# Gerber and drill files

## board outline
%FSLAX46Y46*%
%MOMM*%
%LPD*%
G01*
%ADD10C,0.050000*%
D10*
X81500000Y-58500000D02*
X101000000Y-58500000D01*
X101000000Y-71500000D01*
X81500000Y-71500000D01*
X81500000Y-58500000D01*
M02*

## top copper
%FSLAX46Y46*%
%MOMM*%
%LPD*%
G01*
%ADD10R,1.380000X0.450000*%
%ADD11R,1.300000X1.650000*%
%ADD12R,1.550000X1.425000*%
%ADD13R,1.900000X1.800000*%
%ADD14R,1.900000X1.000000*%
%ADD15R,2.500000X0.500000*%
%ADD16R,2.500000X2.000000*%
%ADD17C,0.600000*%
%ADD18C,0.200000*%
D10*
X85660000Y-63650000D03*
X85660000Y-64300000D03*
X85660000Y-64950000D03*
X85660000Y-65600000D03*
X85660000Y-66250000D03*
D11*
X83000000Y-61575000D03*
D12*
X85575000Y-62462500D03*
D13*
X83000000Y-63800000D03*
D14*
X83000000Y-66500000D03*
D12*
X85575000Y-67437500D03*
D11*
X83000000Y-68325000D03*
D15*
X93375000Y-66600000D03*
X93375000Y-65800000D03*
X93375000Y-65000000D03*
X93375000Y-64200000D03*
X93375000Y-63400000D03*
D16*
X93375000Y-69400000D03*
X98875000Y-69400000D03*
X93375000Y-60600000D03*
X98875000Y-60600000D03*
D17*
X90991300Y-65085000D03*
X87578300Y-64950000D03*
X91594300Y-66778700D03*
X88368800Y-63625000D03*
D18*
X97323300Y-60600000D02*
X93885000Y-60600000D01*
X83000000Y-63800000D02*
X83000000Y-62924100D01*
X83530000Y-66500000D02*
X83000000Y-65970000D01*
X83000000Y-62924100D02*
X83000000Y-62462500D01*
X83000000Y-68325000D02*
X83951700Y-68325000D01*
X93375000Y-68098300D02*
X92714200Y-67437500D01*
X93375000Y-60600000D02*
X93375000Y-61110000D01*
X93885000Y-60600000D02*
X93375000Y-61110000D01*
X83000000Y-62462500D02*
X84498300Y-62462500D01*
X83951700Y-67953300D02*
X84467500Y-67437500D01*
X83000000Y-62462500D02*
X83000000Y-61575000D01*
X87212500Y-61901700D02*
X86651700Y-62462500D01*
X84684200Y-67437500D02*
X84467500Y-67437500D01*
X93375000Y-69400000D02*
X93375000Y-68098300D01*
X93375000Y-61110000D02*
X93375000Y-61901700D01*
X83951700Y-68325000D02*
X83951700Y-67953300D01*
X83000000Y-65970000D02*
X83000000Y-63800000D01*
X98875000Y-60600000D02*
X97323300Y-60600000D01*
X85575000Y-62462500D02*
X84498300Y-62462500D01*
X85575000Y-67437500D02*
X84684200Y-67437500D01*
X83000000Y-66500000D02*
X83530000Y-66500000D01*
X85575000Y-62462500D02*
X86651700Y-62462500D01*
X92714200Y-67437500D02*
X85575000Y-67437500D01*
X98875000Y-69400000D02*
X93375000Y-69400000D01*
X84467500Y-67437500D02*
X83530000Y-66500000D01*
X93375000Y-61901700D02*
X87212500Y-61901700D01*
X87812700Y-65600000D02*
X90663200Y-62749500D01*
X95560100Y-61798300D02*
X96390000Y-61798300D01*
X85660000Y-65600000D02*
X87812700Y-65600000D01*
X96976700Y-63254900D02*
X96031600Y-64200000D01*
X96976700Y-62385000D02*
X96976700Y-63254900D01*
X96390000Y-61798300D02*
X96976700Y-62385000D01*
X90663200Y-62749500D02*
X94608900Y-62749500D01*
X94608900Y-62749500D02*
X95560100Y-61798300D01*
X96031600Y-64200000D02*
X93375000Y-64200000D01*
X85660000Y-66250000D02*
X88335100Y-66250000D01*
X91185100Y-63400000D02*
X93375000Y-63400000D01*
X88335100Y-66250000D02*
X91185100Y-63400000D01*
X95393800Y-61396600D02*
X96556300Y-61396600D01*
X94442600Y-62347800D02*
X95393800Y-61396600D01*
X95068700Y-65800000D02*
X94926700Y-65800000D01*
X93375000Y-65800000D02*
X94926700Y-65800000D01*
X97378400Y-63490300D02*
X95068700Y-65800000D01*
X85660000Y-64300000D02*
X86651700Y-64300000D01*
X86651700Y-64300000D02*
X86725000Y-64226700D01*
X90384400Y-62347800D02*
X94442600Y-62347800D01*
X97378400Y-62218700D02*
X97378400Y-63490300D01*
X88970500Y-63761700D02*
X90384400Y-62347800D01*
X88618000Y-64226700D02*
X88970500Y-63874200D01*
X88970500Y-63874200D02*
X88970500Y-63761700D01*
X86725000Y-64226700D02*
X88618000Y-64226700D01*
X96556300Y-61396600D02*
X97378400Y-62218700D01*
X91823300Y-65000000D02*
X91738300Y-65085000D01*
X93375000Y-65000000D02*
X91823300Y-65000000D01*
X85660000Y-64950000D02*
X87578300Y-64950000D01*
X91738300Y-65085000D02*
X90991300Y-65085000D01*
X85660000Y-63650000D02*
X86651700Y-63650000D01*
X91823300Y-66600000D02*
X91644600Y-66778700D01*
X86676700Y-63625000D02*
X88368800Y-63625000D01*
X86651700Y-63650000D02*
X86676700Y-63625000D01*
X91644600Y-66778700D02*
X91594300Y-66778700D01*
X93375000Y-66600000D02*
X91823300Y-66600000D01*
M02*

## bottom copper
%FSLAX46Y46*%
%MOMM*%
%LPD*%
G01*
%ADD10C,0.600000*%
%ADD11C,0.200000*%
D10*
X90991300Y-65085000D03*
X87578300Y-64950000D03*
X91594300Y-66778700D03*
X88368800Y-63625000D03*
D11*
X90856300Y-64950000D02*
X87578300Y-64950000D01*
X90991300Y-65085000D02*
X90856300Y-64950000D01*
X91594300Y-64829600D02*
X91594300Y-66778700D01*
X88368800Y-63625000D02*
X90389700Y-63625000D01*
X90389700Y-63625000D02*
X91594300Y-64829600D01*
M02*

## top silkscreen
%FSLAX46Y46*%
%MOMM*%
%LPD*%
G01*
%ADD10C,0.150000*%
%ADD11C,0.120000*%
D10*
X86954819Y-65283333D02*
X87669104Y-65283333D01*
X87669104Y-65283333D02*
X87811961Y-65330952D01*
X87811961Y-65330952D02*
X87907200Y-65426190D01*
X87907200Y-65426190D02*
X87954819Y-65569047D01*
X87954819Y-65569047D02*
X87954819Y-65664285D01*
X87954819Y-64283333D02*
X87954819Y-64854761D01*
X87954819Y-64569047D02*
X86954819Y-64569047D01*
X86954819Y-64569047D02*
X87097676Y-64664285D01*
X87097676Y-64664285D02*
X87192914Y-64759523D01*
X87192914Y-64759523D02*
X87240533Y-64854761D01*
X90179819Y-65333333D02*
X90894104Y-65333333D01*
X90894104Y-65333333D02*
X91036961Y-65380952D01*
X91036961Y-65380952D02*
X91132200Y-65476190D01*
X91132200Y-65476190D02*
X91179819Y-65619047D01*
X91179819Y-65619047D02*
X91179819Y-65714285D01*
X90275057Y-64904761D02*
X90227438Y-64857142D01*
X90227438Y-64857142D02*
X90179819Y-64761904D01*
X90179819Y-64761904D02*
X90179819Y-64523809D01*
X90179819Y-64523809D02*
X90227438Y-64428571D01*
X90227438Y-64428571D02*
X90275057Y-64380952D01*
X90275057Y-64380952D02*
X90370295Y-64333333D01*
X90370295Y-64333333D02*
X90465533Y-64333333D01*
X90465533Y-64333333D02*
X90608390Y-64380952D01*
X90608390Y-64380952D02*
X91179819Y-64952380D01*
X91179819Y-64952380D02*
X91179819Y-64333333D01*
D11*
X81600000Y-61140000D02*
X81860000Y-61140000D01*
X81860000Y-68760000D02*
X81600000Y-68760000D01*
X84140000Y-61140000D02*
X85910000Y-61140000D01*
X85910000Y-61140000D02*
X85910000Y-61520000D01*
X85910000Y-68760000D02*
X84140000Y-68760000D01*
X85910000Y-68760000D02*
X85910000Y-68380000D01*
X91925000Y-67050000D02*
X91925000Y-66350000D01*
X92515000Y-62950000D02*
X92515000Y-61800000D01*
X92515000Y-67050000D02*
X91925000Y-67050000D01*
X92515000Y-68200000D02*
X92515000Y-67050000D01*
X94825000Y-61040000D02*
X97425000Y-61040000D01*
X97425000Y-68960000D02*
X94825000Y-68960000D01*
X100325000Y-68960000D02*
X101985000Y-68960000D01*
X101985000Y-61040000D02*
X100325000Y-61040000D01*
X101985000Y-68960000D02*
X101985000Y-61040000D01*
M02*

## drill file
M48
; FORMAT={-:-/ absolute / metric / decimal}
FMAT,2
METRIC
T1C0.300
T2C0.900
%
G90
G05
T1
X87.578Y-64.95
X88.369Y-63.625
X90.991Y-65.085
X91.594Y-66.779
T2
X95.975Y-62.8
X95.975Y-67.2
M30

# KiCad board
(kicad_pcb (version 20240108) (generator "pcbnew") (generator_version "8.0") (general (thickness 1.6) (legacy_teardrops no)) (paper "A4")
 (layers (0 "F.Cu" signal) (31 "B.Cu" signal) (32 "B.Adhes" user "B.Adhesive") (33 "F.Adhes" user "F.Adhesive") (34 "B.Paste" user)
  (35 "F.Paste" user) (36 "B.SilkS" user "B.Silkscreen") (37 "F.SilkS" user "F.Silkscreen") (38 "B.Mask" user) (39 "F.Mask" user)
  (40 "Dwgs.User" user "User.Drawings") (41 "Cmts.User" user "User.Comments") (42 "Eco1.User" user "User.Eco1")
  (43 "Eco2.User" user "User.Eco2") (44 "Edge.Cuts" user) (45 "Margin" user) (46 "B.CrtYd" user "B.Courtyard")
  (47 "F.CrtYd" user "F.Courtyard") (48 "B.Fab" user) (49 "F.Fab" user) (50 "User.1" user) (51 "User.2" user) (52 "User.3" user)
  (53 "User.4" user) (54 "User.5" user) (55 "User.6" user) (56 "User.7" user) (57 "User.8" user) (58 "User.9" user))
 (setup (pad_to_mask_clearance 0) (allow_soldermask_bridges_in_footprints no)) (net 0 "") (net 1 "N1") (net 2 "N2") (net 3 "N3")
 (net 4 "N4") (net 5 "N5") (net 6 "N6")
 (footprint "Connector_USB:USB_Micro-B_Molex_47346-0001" (layer "F.Cu") (at 84.2 64.95 -90)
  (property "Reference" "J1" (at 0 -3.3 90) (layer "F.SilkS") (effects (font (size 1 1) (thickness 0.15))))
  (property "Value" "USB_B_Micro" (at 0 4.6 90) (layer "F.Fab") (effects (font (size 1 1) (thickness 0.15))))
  (fp_line (start -3.81 2.6) (end -3.81 2.34) (stroke (width 0.12) (type solid)) (layer "F.SilkS"))
  (fp_line (start 3.81 2.34) (end 3.81 2.6) (stroke (width 0.12) (type solid)) (layer "F.SilkS"))
  (fp_line (start -3.81 0.06) (end -3.81 -1.71) (stroke (width 0.12) (type solid)) (layer "F.SilkS"))
  (fp_line (start -3.81 -1.71) (end -3.43 -1.71) (stroke (width 0.12) (type solid)) (layer "F.SilkS"))
  (fp_line (start 3.81 -1.71) (end 3.81 0.06) (stroke (width 0.12) (type solid)) (layer "F.SilkS"))
  (fp_line (start 3.81 -1.71) (end 3.43 -1.71) (stroke (width 0.12) (type solid)) (layer "F.SilkS"))
  (pad "1" smd rect (at -1.3 -1.46 270) (size 0.45 1.38) (layers "F.Cu" "F.Paste" "F.Mask") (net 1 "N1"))
  (pad "2" smd rect (at -0.65 -1.46 270) (size 0.45 1.38) (layers "F.Cu" "F.Paste" "F.Mask") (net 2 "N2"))
  (pad "3" smd rect (at 0 -1.46 270) (size 0.45 1.38) (layers "F.Cu" "F.Paste" "F.Mask") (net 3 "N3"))
  (pad "4" smd rect (at 0.65 -1.46 270) (size 0.45 1.38) (layers "F.Cu" "F.Paste" "F.Mask") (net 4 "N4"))
  (pad "5" smd rect (at 1.3 -1.46 270) (size 0.45 1.38) (layers "F.Cu" "F.Paste" "F.Mask") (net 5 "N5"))
  (pad "6" smd rect (at -3.375 1.2 270) (size 1.65 1.3) (layers "F.Cu" "F.Paste" "F.Mask") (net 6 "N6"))
  (pad "6" smd rect (at -2.4875 -1.375 270) (size 1.425 1.55) (layers "F.Cu" "F.Paste" "F.Mask") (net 6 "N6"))
  (pad "6" smd rect (at -1.15 1.2 270) (size 1.8 1.9) (layers "F.Cu" "F.Paste" "F.Mask") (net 6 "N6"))
  (pad "6" smd rect (at 1.55 1.2 270) (size 1 1.9) (layers "F.Cu" "F.Paste" "F.Mask") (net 6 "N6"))
  (pad "6" smd rect (at 2.4875 -1.375 270) (size 1.425 1.55) (layers "F.Cu" "F.Paste" "F.Mask") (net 6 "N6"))
  (pad "6" smd rect (at 3.375 1.2 270) (size 1.65 1.3) (layers "F.Cu" "F.Paste" "F.Mask") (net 6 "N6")))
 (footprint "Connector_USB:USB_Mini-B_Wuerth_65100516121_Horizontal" (layer "F.Cu") (at 95.975 65 90)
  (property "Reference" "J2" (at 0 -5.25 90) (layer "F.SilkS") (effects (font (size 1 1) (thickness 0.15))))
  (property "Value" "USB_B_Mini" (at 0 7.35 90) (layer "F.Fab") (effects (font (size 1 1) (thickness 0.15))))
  (fp_line (start -2.05 -4.05) (end -1.35 -4.05) (stroke (width 0.12) (type solid)) (layer "F.SilkS"))
  (fp_line (start 2.05 -3.46) (end 3.2 -3.46) (stroke (width 0.12) (type solid)) (layer "F.SilkS"))
  (fp_line (start -2.05 -3.46) (end -2.05 -4.05) (stroke (width 0.12) (type solid)) (layer "F.SilkS"))
  (fp_line (start -3.2 -3.46) (end -2.05 -3.46) (stroke (width 0.12) (type solid)) (layer "F.SilkS"))
  (fp_line (start 3.96 -1.15) (end 3.96 1.45) (stroke (width 0.12) (type solid)) (layer "F.SilkS"))
  (fp_line (start -3.96 1.45) (end -3.96 -1.15) (stroke (width 0.12) (type solid)) (layer "F.SilkS"))
  (fp_line (start -3.96 4.35) (end -3.96 6.01) (stroke (width 0.12) (type solid)) (layer "F.SilkS"))
  (fp_line (start 3.96 6.01) (end 3.96 4.35) (stroke (width 0.12) (type solid)) (layer "F.SilkS"))
  (fp_line (start -3.96 6.01) (end 3.96 6.01) (stroke (width 0.12) (type solid)) (layer "F.SilkS"))
  (pad "" np_thru_hole circle (at -2.2 0 90) (size 0.9 0.9) (drill 0.9) (layers "*.Cu" "*.Mask"))
  (pad "" np_thru_hole circle (at 2.2 0 90) (size 0.9 0.9) (drill 0.9) (layers "*.Cu" "*.Mask"))
  (pad "1" smd rect (at -1.6 -2.6 90) (size 0.5 2.5) (layers "F.Cu" "F.Paste" "F.Mask") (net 1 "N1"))
  (pad "2" smd rect (at -0.8 -2.6 90) (size 0.5 2.5) (layers "F.Cu" "F.Paste" "F.Mask") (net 2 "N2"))
  (pad "3" smd rect (at 0 -2.6 90) (size 0.5 2.5) (layers "F.Cu" "F.Paste" "F.Mask") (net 3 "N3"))
  (pad "4" smd rect (at 0.8 -2.6 90) (size 0.5 2.5) (layers "F.Cu" "F.Paste" "F.Mask") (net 4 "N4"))
  (pad "5" smd rect (at 1.6 -2.6 90) (size 0.5 2.5) (layers "F.Cu" "F.Paste" "F.Mask") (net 5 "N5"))
  (pad "6" smd rect (at -4.4 -2.6 90) (size 2 2.5) (layers "F.Cu" "F.Paste" "F.Mask") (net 6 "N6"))
  (pad "6" smd rect (at -4.4 2.9 90) (size 2 2.5) (layers "F.Cu" "F.Paste" "F.Mask") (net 6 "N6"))
  (pad "6" smd rect (at 4.4 -2.6 90) (size 2 2.5) (layers "F.Cu" "F.Paste" "F.Mask") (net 6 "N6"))
  (pad "6" smd rect (at 4.4 2.9 90) (size 2 2.5) (layers "F.Cu" "F.Paste" "F.Mask") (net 6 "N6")))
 (gr_rect (start 81.5 58.5) (end 101 71.5) (stroke (width 0.05) (type default)) (fill none) (layer "Edge.Cuts"))
 (segment (start 97.3233 60.6) (end 93.885 60.6) (width 0.2) (layer "F.Cu") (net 6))
 (segment (start 83 63.8) (end 83 62.9241) (width 0.2) (layer "F.Cu") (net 6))
 (segment (start 83.53 66.5) (end 83 65.97) (width 0.2) (layer "F.Cu") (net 6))
 (segment (start 83 62.9241) (end 83 62.4625) (width 0.2) (layer "F.Cu") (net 6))
 (segment (start 83 68.325) (end 83.9517 68.325) (width 0.2) (layer "F.Cu") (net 6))
 (segment (start 93.375 68.0983) (end 92.7142 67.4375) (width 0.2) (layer "F.Cu") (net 6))
 (segment (start 93.375 60.6) (end 93.375 61.11) (width 0.2) (layer "F.Cu") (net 6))
 (segment (start 93.885 60.6) (end 93.375 61.11) (width 0.2) (layer "F.Cu") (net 6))
 (segment (start 83 62.4625) (end 84.4983 62.4625) (width 0.2) (layer "F.Cu") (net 6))
 (segment (start 83.9517 67.9533) (end 84.4675 67.4375) (width 0.2) (layer "F.Cu") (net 6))
 (segment (start 83 62.4625) (end 83 61.575) (width 0.2) (layer "F.Cu") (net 6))
 (segment (start 87.2125 61.9017) (end 86.6517 62.4625) (width 0.2) (layer "F.Cu") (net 6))
 (segment (start 84.6842 67.4375) (end 84.4675 67.4375) (width 0.2) (layer "F.Cu") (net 6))
 (segment (start 93.375 69.4) (end 93.375 68.0983) (width 0.2) (layer "F.Cu") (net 6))
 (segment (start 93.375 61.11) (end 93.375 61.9017) (width 0.2) (layer "F.Cu") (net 6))
 (segment (start 83.9517 68.325) (end 83.9517 67.9533) (width 0.2) (layer "F.Cu") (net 6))
 (segment (start 83 65.97) (end 83 63.8) (width 0.2) (layer "F.Cu") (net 6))
 (segment (start 98.875 60.6) (end 97.3233 60.6) (width 0.2) (layer "F.Cu") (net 6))
 (segment (start 85.575 62.4625) (end 84.4983 62.4625) (width 0.2) (layer "F.Cu") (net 6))
 (segment (start 85.575 67.4375) (end 84.6842 67.4375) (width 0.2) (layer "F.Cu") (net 6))
 (segment (start 83 66.5) (end 83.53 66.5) (width 0.2) (layer "F.Cu") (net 6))
 (segment (start 85.575 62.4625) (end 86.6517 62.4625) (width 0.2) (layer "F.Cu") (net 6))
 (segment (start 92.7142 67.4375) (end 85.575 67.4375) (width 0.2) (layer "F.Cu") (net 6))
 (segment (start 98.875 69.4) (end 93.375 69.4) (width 0.2) (layer "F.Cu") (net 6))
 (segment (start 84.4675 67.4375) (end 83.53 66.5) (width 0.2) (layer "F.Cu") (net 6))
 (segment (start 93.375 61.9017) (end 87.2125 61.9017) (width 0.2) (layer "F.Cu") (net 6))
 (segment (start 87.8127 65.6) (end 90.6632 62.7495) (width 0.2) (layer "F.Cu") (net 4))
 (segment (start 95.5601 61.7983) (end 96.39 61.7983) (width 0.2) (layer "F.Cu") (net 4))
 (segment (start 85.66 65.6) (end 87.8127 65.6) (width 0.2) (layer "F.Cu") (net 4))
 (segment (start 96.9767 63.2549) (end 96.0316 64.2) (width 0.2) (layer "F.Cu") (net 4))
 (segment (start 96.9767 62.385) (end 96.9767 63.2549) (width 0.2) (layer "F.Cu") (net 4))
 (segment (start 96.39 61.7983) (end 96.9767 62.385) (width 0.2) (layer "F.Cu") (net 4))
 (segment (start 90.6632 62.7495) (end 94.6089 62.7495) (width 0.2) (layer "F.Cu") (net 4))
 (segment (start 94.6089 62.7495) (end 95.5601 61.7983) (width 0.2) (layer "F.Cu") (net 4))
 (segment (start 96.0316 64.2) (end 93.375 64.2) (width 0.2) (layer "F.Cu") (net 4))
 (segment (start 85.66 66.25) (end 88.3351 66.25) (width 0.2) (layer "F.Cu") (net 5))
 (segment (start 91.1851 63.4) (end 93.375 63.4) (width 0.2) (layer "F.Cu") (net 5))
 (segment (start 88.3351 66.25) (end 91.1851 63.4) (width 0.2) (layer "F.Cu") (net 5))
 (segment (start 95.3938 61.3966) (end 96.5563 61.3966) (width 0.2) (layer "F.Cu") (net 2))
 (segment (start 94.4426 62.3478) (end 95.3938 61.3966) (width 0.2) (layer "F.Cu") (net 2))
 (segment (start 95.0687 65.8) (end 94.9267 65.8) (width 0.2) (layer "F.Cu") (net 2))
 (segment (start 93.375 65.8) (end 94.9267 65.8) (width 0.2) (layer "F.Cu") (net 2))
 (segment (start 97.3784 63.4903) (end 95.0687 65.8) (width 0.2) (layer "F.Cu") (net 2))
 (segment (start 85.66 64.3) (end 86.6517 64.3) (width 0.2) (layer "F.Cu") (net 2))
 (segment (start 86.6517 64.3) (end 86.725 64.2267) (width 0.2) (layer "F.Cu") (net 2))
 (segment (start 90.3844 62.3478) (end 94.4426 62.3478) (width 0.2) (layer "F.Cu") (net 2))
 (segment (start 97.3784 62.2187) (end 97.3784 63.4903) (width 0.2) (layer "F.Cu") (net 2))
 (segment (start 88.9705 63.7617) (end 90.3844 62.3478) (width 0.2) (layer "F.Cu") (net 2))
 (segment (start 88.618 64.2267) (end 88.9705 63.8742) (width 0.2) (layer "F.Cu") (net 2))
 (segment (start 88.9705 63.8742) (end 88.9705 63.7617) (width 0.2) (layer "F.Cu") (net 2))
 (segment (start 86.725 64.2267) (end 88.618 64.2267) (width 0.2) (layer "F.Cu") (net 2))
 (segment (start 96.5563 61.3966) (end 97.3784 62.2187) (width 0.2) (layer "F.Cu") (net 2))
 (segment (start 91.8233 65) (end 91.7383 65.085) (width 0.2) (layer "F.Cu") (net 3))
 (segment (start 93.375 65) (end 91.8233 65) (width 0.2) (layer "F.Cu") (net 3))
 (segment (start 85.66 64.95) (end 87.5783 64.95) (width 0.2) (layer "F.Cu") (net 3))
 (segment (start 91.7383 65.085) (end 90.9913 65.085) (width 0.2) (layer "F.Cu") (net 3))
 (via (at 90.9913 65.085) (size 0.6) (drill 0.3) (layers "F.Cu" "B.Cu") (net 3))
 (via (at 87.5783 64.95) (size 0.6) (drill 0.3) (layers "F.Cu" "B.Cu") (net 3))
 (segment (start 90.8563 64.95) (end 87.5783 64.95) (width 0.2) (layer "B.Cu") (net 3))
 (segment (start 90.9913 65.085) (end 90.8563 64.95) (width 0.2) (layer "B.Cu") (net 3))
 (segment (start 85.66 63.65) (end 86.6517 63.65) (width 0.2) (layer "F.Cu") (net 1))
 (segment (start 91.8233 66.6) (end 91.6446 66.7787) (width 0.2) (layer "F.Cu") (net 1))
 (segment (start 86.6767 63.625) (end 88.3688 63.625) (width 0.2) (layer "F.Cu") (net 1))
 (segment (start 86.6517 63.65) (end 86.6767 63.625) (width 0.2) (layer "F.Cu") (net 1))
 (segment (start 91.6446 66.7787) (end 91.5943 66.7787) (width 0.2) (layer "F.Cu") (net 1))
 (segment (start 93.375 66.6) (end 91.8233 66.6) (width 0.2) (layer "F.Cu") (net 1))
 (via (at 91.5943 66.7787) (size 0.6) (drill 0.3) (layers "F.Cu" "B.Cu") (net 1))
 (via (at 88.3688 63.625) (size 0.6) (drill 0.3) (layers "F.Cu" "B.Cu") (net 1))
 (segment (start 91.5943 64.8296) (end 91.5943 66.7787) (width 0.2) (layer "B.Cu") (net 1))
 (segment (start 88.3688 63.625) (end 90.3897 63.625) (width 0.2) (layer "B.Cu") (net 1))
 (segment (start 90.3897 63.625) (end 91.5943 64.8296) (width 0.2) (layer "B.Cu") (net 1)))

